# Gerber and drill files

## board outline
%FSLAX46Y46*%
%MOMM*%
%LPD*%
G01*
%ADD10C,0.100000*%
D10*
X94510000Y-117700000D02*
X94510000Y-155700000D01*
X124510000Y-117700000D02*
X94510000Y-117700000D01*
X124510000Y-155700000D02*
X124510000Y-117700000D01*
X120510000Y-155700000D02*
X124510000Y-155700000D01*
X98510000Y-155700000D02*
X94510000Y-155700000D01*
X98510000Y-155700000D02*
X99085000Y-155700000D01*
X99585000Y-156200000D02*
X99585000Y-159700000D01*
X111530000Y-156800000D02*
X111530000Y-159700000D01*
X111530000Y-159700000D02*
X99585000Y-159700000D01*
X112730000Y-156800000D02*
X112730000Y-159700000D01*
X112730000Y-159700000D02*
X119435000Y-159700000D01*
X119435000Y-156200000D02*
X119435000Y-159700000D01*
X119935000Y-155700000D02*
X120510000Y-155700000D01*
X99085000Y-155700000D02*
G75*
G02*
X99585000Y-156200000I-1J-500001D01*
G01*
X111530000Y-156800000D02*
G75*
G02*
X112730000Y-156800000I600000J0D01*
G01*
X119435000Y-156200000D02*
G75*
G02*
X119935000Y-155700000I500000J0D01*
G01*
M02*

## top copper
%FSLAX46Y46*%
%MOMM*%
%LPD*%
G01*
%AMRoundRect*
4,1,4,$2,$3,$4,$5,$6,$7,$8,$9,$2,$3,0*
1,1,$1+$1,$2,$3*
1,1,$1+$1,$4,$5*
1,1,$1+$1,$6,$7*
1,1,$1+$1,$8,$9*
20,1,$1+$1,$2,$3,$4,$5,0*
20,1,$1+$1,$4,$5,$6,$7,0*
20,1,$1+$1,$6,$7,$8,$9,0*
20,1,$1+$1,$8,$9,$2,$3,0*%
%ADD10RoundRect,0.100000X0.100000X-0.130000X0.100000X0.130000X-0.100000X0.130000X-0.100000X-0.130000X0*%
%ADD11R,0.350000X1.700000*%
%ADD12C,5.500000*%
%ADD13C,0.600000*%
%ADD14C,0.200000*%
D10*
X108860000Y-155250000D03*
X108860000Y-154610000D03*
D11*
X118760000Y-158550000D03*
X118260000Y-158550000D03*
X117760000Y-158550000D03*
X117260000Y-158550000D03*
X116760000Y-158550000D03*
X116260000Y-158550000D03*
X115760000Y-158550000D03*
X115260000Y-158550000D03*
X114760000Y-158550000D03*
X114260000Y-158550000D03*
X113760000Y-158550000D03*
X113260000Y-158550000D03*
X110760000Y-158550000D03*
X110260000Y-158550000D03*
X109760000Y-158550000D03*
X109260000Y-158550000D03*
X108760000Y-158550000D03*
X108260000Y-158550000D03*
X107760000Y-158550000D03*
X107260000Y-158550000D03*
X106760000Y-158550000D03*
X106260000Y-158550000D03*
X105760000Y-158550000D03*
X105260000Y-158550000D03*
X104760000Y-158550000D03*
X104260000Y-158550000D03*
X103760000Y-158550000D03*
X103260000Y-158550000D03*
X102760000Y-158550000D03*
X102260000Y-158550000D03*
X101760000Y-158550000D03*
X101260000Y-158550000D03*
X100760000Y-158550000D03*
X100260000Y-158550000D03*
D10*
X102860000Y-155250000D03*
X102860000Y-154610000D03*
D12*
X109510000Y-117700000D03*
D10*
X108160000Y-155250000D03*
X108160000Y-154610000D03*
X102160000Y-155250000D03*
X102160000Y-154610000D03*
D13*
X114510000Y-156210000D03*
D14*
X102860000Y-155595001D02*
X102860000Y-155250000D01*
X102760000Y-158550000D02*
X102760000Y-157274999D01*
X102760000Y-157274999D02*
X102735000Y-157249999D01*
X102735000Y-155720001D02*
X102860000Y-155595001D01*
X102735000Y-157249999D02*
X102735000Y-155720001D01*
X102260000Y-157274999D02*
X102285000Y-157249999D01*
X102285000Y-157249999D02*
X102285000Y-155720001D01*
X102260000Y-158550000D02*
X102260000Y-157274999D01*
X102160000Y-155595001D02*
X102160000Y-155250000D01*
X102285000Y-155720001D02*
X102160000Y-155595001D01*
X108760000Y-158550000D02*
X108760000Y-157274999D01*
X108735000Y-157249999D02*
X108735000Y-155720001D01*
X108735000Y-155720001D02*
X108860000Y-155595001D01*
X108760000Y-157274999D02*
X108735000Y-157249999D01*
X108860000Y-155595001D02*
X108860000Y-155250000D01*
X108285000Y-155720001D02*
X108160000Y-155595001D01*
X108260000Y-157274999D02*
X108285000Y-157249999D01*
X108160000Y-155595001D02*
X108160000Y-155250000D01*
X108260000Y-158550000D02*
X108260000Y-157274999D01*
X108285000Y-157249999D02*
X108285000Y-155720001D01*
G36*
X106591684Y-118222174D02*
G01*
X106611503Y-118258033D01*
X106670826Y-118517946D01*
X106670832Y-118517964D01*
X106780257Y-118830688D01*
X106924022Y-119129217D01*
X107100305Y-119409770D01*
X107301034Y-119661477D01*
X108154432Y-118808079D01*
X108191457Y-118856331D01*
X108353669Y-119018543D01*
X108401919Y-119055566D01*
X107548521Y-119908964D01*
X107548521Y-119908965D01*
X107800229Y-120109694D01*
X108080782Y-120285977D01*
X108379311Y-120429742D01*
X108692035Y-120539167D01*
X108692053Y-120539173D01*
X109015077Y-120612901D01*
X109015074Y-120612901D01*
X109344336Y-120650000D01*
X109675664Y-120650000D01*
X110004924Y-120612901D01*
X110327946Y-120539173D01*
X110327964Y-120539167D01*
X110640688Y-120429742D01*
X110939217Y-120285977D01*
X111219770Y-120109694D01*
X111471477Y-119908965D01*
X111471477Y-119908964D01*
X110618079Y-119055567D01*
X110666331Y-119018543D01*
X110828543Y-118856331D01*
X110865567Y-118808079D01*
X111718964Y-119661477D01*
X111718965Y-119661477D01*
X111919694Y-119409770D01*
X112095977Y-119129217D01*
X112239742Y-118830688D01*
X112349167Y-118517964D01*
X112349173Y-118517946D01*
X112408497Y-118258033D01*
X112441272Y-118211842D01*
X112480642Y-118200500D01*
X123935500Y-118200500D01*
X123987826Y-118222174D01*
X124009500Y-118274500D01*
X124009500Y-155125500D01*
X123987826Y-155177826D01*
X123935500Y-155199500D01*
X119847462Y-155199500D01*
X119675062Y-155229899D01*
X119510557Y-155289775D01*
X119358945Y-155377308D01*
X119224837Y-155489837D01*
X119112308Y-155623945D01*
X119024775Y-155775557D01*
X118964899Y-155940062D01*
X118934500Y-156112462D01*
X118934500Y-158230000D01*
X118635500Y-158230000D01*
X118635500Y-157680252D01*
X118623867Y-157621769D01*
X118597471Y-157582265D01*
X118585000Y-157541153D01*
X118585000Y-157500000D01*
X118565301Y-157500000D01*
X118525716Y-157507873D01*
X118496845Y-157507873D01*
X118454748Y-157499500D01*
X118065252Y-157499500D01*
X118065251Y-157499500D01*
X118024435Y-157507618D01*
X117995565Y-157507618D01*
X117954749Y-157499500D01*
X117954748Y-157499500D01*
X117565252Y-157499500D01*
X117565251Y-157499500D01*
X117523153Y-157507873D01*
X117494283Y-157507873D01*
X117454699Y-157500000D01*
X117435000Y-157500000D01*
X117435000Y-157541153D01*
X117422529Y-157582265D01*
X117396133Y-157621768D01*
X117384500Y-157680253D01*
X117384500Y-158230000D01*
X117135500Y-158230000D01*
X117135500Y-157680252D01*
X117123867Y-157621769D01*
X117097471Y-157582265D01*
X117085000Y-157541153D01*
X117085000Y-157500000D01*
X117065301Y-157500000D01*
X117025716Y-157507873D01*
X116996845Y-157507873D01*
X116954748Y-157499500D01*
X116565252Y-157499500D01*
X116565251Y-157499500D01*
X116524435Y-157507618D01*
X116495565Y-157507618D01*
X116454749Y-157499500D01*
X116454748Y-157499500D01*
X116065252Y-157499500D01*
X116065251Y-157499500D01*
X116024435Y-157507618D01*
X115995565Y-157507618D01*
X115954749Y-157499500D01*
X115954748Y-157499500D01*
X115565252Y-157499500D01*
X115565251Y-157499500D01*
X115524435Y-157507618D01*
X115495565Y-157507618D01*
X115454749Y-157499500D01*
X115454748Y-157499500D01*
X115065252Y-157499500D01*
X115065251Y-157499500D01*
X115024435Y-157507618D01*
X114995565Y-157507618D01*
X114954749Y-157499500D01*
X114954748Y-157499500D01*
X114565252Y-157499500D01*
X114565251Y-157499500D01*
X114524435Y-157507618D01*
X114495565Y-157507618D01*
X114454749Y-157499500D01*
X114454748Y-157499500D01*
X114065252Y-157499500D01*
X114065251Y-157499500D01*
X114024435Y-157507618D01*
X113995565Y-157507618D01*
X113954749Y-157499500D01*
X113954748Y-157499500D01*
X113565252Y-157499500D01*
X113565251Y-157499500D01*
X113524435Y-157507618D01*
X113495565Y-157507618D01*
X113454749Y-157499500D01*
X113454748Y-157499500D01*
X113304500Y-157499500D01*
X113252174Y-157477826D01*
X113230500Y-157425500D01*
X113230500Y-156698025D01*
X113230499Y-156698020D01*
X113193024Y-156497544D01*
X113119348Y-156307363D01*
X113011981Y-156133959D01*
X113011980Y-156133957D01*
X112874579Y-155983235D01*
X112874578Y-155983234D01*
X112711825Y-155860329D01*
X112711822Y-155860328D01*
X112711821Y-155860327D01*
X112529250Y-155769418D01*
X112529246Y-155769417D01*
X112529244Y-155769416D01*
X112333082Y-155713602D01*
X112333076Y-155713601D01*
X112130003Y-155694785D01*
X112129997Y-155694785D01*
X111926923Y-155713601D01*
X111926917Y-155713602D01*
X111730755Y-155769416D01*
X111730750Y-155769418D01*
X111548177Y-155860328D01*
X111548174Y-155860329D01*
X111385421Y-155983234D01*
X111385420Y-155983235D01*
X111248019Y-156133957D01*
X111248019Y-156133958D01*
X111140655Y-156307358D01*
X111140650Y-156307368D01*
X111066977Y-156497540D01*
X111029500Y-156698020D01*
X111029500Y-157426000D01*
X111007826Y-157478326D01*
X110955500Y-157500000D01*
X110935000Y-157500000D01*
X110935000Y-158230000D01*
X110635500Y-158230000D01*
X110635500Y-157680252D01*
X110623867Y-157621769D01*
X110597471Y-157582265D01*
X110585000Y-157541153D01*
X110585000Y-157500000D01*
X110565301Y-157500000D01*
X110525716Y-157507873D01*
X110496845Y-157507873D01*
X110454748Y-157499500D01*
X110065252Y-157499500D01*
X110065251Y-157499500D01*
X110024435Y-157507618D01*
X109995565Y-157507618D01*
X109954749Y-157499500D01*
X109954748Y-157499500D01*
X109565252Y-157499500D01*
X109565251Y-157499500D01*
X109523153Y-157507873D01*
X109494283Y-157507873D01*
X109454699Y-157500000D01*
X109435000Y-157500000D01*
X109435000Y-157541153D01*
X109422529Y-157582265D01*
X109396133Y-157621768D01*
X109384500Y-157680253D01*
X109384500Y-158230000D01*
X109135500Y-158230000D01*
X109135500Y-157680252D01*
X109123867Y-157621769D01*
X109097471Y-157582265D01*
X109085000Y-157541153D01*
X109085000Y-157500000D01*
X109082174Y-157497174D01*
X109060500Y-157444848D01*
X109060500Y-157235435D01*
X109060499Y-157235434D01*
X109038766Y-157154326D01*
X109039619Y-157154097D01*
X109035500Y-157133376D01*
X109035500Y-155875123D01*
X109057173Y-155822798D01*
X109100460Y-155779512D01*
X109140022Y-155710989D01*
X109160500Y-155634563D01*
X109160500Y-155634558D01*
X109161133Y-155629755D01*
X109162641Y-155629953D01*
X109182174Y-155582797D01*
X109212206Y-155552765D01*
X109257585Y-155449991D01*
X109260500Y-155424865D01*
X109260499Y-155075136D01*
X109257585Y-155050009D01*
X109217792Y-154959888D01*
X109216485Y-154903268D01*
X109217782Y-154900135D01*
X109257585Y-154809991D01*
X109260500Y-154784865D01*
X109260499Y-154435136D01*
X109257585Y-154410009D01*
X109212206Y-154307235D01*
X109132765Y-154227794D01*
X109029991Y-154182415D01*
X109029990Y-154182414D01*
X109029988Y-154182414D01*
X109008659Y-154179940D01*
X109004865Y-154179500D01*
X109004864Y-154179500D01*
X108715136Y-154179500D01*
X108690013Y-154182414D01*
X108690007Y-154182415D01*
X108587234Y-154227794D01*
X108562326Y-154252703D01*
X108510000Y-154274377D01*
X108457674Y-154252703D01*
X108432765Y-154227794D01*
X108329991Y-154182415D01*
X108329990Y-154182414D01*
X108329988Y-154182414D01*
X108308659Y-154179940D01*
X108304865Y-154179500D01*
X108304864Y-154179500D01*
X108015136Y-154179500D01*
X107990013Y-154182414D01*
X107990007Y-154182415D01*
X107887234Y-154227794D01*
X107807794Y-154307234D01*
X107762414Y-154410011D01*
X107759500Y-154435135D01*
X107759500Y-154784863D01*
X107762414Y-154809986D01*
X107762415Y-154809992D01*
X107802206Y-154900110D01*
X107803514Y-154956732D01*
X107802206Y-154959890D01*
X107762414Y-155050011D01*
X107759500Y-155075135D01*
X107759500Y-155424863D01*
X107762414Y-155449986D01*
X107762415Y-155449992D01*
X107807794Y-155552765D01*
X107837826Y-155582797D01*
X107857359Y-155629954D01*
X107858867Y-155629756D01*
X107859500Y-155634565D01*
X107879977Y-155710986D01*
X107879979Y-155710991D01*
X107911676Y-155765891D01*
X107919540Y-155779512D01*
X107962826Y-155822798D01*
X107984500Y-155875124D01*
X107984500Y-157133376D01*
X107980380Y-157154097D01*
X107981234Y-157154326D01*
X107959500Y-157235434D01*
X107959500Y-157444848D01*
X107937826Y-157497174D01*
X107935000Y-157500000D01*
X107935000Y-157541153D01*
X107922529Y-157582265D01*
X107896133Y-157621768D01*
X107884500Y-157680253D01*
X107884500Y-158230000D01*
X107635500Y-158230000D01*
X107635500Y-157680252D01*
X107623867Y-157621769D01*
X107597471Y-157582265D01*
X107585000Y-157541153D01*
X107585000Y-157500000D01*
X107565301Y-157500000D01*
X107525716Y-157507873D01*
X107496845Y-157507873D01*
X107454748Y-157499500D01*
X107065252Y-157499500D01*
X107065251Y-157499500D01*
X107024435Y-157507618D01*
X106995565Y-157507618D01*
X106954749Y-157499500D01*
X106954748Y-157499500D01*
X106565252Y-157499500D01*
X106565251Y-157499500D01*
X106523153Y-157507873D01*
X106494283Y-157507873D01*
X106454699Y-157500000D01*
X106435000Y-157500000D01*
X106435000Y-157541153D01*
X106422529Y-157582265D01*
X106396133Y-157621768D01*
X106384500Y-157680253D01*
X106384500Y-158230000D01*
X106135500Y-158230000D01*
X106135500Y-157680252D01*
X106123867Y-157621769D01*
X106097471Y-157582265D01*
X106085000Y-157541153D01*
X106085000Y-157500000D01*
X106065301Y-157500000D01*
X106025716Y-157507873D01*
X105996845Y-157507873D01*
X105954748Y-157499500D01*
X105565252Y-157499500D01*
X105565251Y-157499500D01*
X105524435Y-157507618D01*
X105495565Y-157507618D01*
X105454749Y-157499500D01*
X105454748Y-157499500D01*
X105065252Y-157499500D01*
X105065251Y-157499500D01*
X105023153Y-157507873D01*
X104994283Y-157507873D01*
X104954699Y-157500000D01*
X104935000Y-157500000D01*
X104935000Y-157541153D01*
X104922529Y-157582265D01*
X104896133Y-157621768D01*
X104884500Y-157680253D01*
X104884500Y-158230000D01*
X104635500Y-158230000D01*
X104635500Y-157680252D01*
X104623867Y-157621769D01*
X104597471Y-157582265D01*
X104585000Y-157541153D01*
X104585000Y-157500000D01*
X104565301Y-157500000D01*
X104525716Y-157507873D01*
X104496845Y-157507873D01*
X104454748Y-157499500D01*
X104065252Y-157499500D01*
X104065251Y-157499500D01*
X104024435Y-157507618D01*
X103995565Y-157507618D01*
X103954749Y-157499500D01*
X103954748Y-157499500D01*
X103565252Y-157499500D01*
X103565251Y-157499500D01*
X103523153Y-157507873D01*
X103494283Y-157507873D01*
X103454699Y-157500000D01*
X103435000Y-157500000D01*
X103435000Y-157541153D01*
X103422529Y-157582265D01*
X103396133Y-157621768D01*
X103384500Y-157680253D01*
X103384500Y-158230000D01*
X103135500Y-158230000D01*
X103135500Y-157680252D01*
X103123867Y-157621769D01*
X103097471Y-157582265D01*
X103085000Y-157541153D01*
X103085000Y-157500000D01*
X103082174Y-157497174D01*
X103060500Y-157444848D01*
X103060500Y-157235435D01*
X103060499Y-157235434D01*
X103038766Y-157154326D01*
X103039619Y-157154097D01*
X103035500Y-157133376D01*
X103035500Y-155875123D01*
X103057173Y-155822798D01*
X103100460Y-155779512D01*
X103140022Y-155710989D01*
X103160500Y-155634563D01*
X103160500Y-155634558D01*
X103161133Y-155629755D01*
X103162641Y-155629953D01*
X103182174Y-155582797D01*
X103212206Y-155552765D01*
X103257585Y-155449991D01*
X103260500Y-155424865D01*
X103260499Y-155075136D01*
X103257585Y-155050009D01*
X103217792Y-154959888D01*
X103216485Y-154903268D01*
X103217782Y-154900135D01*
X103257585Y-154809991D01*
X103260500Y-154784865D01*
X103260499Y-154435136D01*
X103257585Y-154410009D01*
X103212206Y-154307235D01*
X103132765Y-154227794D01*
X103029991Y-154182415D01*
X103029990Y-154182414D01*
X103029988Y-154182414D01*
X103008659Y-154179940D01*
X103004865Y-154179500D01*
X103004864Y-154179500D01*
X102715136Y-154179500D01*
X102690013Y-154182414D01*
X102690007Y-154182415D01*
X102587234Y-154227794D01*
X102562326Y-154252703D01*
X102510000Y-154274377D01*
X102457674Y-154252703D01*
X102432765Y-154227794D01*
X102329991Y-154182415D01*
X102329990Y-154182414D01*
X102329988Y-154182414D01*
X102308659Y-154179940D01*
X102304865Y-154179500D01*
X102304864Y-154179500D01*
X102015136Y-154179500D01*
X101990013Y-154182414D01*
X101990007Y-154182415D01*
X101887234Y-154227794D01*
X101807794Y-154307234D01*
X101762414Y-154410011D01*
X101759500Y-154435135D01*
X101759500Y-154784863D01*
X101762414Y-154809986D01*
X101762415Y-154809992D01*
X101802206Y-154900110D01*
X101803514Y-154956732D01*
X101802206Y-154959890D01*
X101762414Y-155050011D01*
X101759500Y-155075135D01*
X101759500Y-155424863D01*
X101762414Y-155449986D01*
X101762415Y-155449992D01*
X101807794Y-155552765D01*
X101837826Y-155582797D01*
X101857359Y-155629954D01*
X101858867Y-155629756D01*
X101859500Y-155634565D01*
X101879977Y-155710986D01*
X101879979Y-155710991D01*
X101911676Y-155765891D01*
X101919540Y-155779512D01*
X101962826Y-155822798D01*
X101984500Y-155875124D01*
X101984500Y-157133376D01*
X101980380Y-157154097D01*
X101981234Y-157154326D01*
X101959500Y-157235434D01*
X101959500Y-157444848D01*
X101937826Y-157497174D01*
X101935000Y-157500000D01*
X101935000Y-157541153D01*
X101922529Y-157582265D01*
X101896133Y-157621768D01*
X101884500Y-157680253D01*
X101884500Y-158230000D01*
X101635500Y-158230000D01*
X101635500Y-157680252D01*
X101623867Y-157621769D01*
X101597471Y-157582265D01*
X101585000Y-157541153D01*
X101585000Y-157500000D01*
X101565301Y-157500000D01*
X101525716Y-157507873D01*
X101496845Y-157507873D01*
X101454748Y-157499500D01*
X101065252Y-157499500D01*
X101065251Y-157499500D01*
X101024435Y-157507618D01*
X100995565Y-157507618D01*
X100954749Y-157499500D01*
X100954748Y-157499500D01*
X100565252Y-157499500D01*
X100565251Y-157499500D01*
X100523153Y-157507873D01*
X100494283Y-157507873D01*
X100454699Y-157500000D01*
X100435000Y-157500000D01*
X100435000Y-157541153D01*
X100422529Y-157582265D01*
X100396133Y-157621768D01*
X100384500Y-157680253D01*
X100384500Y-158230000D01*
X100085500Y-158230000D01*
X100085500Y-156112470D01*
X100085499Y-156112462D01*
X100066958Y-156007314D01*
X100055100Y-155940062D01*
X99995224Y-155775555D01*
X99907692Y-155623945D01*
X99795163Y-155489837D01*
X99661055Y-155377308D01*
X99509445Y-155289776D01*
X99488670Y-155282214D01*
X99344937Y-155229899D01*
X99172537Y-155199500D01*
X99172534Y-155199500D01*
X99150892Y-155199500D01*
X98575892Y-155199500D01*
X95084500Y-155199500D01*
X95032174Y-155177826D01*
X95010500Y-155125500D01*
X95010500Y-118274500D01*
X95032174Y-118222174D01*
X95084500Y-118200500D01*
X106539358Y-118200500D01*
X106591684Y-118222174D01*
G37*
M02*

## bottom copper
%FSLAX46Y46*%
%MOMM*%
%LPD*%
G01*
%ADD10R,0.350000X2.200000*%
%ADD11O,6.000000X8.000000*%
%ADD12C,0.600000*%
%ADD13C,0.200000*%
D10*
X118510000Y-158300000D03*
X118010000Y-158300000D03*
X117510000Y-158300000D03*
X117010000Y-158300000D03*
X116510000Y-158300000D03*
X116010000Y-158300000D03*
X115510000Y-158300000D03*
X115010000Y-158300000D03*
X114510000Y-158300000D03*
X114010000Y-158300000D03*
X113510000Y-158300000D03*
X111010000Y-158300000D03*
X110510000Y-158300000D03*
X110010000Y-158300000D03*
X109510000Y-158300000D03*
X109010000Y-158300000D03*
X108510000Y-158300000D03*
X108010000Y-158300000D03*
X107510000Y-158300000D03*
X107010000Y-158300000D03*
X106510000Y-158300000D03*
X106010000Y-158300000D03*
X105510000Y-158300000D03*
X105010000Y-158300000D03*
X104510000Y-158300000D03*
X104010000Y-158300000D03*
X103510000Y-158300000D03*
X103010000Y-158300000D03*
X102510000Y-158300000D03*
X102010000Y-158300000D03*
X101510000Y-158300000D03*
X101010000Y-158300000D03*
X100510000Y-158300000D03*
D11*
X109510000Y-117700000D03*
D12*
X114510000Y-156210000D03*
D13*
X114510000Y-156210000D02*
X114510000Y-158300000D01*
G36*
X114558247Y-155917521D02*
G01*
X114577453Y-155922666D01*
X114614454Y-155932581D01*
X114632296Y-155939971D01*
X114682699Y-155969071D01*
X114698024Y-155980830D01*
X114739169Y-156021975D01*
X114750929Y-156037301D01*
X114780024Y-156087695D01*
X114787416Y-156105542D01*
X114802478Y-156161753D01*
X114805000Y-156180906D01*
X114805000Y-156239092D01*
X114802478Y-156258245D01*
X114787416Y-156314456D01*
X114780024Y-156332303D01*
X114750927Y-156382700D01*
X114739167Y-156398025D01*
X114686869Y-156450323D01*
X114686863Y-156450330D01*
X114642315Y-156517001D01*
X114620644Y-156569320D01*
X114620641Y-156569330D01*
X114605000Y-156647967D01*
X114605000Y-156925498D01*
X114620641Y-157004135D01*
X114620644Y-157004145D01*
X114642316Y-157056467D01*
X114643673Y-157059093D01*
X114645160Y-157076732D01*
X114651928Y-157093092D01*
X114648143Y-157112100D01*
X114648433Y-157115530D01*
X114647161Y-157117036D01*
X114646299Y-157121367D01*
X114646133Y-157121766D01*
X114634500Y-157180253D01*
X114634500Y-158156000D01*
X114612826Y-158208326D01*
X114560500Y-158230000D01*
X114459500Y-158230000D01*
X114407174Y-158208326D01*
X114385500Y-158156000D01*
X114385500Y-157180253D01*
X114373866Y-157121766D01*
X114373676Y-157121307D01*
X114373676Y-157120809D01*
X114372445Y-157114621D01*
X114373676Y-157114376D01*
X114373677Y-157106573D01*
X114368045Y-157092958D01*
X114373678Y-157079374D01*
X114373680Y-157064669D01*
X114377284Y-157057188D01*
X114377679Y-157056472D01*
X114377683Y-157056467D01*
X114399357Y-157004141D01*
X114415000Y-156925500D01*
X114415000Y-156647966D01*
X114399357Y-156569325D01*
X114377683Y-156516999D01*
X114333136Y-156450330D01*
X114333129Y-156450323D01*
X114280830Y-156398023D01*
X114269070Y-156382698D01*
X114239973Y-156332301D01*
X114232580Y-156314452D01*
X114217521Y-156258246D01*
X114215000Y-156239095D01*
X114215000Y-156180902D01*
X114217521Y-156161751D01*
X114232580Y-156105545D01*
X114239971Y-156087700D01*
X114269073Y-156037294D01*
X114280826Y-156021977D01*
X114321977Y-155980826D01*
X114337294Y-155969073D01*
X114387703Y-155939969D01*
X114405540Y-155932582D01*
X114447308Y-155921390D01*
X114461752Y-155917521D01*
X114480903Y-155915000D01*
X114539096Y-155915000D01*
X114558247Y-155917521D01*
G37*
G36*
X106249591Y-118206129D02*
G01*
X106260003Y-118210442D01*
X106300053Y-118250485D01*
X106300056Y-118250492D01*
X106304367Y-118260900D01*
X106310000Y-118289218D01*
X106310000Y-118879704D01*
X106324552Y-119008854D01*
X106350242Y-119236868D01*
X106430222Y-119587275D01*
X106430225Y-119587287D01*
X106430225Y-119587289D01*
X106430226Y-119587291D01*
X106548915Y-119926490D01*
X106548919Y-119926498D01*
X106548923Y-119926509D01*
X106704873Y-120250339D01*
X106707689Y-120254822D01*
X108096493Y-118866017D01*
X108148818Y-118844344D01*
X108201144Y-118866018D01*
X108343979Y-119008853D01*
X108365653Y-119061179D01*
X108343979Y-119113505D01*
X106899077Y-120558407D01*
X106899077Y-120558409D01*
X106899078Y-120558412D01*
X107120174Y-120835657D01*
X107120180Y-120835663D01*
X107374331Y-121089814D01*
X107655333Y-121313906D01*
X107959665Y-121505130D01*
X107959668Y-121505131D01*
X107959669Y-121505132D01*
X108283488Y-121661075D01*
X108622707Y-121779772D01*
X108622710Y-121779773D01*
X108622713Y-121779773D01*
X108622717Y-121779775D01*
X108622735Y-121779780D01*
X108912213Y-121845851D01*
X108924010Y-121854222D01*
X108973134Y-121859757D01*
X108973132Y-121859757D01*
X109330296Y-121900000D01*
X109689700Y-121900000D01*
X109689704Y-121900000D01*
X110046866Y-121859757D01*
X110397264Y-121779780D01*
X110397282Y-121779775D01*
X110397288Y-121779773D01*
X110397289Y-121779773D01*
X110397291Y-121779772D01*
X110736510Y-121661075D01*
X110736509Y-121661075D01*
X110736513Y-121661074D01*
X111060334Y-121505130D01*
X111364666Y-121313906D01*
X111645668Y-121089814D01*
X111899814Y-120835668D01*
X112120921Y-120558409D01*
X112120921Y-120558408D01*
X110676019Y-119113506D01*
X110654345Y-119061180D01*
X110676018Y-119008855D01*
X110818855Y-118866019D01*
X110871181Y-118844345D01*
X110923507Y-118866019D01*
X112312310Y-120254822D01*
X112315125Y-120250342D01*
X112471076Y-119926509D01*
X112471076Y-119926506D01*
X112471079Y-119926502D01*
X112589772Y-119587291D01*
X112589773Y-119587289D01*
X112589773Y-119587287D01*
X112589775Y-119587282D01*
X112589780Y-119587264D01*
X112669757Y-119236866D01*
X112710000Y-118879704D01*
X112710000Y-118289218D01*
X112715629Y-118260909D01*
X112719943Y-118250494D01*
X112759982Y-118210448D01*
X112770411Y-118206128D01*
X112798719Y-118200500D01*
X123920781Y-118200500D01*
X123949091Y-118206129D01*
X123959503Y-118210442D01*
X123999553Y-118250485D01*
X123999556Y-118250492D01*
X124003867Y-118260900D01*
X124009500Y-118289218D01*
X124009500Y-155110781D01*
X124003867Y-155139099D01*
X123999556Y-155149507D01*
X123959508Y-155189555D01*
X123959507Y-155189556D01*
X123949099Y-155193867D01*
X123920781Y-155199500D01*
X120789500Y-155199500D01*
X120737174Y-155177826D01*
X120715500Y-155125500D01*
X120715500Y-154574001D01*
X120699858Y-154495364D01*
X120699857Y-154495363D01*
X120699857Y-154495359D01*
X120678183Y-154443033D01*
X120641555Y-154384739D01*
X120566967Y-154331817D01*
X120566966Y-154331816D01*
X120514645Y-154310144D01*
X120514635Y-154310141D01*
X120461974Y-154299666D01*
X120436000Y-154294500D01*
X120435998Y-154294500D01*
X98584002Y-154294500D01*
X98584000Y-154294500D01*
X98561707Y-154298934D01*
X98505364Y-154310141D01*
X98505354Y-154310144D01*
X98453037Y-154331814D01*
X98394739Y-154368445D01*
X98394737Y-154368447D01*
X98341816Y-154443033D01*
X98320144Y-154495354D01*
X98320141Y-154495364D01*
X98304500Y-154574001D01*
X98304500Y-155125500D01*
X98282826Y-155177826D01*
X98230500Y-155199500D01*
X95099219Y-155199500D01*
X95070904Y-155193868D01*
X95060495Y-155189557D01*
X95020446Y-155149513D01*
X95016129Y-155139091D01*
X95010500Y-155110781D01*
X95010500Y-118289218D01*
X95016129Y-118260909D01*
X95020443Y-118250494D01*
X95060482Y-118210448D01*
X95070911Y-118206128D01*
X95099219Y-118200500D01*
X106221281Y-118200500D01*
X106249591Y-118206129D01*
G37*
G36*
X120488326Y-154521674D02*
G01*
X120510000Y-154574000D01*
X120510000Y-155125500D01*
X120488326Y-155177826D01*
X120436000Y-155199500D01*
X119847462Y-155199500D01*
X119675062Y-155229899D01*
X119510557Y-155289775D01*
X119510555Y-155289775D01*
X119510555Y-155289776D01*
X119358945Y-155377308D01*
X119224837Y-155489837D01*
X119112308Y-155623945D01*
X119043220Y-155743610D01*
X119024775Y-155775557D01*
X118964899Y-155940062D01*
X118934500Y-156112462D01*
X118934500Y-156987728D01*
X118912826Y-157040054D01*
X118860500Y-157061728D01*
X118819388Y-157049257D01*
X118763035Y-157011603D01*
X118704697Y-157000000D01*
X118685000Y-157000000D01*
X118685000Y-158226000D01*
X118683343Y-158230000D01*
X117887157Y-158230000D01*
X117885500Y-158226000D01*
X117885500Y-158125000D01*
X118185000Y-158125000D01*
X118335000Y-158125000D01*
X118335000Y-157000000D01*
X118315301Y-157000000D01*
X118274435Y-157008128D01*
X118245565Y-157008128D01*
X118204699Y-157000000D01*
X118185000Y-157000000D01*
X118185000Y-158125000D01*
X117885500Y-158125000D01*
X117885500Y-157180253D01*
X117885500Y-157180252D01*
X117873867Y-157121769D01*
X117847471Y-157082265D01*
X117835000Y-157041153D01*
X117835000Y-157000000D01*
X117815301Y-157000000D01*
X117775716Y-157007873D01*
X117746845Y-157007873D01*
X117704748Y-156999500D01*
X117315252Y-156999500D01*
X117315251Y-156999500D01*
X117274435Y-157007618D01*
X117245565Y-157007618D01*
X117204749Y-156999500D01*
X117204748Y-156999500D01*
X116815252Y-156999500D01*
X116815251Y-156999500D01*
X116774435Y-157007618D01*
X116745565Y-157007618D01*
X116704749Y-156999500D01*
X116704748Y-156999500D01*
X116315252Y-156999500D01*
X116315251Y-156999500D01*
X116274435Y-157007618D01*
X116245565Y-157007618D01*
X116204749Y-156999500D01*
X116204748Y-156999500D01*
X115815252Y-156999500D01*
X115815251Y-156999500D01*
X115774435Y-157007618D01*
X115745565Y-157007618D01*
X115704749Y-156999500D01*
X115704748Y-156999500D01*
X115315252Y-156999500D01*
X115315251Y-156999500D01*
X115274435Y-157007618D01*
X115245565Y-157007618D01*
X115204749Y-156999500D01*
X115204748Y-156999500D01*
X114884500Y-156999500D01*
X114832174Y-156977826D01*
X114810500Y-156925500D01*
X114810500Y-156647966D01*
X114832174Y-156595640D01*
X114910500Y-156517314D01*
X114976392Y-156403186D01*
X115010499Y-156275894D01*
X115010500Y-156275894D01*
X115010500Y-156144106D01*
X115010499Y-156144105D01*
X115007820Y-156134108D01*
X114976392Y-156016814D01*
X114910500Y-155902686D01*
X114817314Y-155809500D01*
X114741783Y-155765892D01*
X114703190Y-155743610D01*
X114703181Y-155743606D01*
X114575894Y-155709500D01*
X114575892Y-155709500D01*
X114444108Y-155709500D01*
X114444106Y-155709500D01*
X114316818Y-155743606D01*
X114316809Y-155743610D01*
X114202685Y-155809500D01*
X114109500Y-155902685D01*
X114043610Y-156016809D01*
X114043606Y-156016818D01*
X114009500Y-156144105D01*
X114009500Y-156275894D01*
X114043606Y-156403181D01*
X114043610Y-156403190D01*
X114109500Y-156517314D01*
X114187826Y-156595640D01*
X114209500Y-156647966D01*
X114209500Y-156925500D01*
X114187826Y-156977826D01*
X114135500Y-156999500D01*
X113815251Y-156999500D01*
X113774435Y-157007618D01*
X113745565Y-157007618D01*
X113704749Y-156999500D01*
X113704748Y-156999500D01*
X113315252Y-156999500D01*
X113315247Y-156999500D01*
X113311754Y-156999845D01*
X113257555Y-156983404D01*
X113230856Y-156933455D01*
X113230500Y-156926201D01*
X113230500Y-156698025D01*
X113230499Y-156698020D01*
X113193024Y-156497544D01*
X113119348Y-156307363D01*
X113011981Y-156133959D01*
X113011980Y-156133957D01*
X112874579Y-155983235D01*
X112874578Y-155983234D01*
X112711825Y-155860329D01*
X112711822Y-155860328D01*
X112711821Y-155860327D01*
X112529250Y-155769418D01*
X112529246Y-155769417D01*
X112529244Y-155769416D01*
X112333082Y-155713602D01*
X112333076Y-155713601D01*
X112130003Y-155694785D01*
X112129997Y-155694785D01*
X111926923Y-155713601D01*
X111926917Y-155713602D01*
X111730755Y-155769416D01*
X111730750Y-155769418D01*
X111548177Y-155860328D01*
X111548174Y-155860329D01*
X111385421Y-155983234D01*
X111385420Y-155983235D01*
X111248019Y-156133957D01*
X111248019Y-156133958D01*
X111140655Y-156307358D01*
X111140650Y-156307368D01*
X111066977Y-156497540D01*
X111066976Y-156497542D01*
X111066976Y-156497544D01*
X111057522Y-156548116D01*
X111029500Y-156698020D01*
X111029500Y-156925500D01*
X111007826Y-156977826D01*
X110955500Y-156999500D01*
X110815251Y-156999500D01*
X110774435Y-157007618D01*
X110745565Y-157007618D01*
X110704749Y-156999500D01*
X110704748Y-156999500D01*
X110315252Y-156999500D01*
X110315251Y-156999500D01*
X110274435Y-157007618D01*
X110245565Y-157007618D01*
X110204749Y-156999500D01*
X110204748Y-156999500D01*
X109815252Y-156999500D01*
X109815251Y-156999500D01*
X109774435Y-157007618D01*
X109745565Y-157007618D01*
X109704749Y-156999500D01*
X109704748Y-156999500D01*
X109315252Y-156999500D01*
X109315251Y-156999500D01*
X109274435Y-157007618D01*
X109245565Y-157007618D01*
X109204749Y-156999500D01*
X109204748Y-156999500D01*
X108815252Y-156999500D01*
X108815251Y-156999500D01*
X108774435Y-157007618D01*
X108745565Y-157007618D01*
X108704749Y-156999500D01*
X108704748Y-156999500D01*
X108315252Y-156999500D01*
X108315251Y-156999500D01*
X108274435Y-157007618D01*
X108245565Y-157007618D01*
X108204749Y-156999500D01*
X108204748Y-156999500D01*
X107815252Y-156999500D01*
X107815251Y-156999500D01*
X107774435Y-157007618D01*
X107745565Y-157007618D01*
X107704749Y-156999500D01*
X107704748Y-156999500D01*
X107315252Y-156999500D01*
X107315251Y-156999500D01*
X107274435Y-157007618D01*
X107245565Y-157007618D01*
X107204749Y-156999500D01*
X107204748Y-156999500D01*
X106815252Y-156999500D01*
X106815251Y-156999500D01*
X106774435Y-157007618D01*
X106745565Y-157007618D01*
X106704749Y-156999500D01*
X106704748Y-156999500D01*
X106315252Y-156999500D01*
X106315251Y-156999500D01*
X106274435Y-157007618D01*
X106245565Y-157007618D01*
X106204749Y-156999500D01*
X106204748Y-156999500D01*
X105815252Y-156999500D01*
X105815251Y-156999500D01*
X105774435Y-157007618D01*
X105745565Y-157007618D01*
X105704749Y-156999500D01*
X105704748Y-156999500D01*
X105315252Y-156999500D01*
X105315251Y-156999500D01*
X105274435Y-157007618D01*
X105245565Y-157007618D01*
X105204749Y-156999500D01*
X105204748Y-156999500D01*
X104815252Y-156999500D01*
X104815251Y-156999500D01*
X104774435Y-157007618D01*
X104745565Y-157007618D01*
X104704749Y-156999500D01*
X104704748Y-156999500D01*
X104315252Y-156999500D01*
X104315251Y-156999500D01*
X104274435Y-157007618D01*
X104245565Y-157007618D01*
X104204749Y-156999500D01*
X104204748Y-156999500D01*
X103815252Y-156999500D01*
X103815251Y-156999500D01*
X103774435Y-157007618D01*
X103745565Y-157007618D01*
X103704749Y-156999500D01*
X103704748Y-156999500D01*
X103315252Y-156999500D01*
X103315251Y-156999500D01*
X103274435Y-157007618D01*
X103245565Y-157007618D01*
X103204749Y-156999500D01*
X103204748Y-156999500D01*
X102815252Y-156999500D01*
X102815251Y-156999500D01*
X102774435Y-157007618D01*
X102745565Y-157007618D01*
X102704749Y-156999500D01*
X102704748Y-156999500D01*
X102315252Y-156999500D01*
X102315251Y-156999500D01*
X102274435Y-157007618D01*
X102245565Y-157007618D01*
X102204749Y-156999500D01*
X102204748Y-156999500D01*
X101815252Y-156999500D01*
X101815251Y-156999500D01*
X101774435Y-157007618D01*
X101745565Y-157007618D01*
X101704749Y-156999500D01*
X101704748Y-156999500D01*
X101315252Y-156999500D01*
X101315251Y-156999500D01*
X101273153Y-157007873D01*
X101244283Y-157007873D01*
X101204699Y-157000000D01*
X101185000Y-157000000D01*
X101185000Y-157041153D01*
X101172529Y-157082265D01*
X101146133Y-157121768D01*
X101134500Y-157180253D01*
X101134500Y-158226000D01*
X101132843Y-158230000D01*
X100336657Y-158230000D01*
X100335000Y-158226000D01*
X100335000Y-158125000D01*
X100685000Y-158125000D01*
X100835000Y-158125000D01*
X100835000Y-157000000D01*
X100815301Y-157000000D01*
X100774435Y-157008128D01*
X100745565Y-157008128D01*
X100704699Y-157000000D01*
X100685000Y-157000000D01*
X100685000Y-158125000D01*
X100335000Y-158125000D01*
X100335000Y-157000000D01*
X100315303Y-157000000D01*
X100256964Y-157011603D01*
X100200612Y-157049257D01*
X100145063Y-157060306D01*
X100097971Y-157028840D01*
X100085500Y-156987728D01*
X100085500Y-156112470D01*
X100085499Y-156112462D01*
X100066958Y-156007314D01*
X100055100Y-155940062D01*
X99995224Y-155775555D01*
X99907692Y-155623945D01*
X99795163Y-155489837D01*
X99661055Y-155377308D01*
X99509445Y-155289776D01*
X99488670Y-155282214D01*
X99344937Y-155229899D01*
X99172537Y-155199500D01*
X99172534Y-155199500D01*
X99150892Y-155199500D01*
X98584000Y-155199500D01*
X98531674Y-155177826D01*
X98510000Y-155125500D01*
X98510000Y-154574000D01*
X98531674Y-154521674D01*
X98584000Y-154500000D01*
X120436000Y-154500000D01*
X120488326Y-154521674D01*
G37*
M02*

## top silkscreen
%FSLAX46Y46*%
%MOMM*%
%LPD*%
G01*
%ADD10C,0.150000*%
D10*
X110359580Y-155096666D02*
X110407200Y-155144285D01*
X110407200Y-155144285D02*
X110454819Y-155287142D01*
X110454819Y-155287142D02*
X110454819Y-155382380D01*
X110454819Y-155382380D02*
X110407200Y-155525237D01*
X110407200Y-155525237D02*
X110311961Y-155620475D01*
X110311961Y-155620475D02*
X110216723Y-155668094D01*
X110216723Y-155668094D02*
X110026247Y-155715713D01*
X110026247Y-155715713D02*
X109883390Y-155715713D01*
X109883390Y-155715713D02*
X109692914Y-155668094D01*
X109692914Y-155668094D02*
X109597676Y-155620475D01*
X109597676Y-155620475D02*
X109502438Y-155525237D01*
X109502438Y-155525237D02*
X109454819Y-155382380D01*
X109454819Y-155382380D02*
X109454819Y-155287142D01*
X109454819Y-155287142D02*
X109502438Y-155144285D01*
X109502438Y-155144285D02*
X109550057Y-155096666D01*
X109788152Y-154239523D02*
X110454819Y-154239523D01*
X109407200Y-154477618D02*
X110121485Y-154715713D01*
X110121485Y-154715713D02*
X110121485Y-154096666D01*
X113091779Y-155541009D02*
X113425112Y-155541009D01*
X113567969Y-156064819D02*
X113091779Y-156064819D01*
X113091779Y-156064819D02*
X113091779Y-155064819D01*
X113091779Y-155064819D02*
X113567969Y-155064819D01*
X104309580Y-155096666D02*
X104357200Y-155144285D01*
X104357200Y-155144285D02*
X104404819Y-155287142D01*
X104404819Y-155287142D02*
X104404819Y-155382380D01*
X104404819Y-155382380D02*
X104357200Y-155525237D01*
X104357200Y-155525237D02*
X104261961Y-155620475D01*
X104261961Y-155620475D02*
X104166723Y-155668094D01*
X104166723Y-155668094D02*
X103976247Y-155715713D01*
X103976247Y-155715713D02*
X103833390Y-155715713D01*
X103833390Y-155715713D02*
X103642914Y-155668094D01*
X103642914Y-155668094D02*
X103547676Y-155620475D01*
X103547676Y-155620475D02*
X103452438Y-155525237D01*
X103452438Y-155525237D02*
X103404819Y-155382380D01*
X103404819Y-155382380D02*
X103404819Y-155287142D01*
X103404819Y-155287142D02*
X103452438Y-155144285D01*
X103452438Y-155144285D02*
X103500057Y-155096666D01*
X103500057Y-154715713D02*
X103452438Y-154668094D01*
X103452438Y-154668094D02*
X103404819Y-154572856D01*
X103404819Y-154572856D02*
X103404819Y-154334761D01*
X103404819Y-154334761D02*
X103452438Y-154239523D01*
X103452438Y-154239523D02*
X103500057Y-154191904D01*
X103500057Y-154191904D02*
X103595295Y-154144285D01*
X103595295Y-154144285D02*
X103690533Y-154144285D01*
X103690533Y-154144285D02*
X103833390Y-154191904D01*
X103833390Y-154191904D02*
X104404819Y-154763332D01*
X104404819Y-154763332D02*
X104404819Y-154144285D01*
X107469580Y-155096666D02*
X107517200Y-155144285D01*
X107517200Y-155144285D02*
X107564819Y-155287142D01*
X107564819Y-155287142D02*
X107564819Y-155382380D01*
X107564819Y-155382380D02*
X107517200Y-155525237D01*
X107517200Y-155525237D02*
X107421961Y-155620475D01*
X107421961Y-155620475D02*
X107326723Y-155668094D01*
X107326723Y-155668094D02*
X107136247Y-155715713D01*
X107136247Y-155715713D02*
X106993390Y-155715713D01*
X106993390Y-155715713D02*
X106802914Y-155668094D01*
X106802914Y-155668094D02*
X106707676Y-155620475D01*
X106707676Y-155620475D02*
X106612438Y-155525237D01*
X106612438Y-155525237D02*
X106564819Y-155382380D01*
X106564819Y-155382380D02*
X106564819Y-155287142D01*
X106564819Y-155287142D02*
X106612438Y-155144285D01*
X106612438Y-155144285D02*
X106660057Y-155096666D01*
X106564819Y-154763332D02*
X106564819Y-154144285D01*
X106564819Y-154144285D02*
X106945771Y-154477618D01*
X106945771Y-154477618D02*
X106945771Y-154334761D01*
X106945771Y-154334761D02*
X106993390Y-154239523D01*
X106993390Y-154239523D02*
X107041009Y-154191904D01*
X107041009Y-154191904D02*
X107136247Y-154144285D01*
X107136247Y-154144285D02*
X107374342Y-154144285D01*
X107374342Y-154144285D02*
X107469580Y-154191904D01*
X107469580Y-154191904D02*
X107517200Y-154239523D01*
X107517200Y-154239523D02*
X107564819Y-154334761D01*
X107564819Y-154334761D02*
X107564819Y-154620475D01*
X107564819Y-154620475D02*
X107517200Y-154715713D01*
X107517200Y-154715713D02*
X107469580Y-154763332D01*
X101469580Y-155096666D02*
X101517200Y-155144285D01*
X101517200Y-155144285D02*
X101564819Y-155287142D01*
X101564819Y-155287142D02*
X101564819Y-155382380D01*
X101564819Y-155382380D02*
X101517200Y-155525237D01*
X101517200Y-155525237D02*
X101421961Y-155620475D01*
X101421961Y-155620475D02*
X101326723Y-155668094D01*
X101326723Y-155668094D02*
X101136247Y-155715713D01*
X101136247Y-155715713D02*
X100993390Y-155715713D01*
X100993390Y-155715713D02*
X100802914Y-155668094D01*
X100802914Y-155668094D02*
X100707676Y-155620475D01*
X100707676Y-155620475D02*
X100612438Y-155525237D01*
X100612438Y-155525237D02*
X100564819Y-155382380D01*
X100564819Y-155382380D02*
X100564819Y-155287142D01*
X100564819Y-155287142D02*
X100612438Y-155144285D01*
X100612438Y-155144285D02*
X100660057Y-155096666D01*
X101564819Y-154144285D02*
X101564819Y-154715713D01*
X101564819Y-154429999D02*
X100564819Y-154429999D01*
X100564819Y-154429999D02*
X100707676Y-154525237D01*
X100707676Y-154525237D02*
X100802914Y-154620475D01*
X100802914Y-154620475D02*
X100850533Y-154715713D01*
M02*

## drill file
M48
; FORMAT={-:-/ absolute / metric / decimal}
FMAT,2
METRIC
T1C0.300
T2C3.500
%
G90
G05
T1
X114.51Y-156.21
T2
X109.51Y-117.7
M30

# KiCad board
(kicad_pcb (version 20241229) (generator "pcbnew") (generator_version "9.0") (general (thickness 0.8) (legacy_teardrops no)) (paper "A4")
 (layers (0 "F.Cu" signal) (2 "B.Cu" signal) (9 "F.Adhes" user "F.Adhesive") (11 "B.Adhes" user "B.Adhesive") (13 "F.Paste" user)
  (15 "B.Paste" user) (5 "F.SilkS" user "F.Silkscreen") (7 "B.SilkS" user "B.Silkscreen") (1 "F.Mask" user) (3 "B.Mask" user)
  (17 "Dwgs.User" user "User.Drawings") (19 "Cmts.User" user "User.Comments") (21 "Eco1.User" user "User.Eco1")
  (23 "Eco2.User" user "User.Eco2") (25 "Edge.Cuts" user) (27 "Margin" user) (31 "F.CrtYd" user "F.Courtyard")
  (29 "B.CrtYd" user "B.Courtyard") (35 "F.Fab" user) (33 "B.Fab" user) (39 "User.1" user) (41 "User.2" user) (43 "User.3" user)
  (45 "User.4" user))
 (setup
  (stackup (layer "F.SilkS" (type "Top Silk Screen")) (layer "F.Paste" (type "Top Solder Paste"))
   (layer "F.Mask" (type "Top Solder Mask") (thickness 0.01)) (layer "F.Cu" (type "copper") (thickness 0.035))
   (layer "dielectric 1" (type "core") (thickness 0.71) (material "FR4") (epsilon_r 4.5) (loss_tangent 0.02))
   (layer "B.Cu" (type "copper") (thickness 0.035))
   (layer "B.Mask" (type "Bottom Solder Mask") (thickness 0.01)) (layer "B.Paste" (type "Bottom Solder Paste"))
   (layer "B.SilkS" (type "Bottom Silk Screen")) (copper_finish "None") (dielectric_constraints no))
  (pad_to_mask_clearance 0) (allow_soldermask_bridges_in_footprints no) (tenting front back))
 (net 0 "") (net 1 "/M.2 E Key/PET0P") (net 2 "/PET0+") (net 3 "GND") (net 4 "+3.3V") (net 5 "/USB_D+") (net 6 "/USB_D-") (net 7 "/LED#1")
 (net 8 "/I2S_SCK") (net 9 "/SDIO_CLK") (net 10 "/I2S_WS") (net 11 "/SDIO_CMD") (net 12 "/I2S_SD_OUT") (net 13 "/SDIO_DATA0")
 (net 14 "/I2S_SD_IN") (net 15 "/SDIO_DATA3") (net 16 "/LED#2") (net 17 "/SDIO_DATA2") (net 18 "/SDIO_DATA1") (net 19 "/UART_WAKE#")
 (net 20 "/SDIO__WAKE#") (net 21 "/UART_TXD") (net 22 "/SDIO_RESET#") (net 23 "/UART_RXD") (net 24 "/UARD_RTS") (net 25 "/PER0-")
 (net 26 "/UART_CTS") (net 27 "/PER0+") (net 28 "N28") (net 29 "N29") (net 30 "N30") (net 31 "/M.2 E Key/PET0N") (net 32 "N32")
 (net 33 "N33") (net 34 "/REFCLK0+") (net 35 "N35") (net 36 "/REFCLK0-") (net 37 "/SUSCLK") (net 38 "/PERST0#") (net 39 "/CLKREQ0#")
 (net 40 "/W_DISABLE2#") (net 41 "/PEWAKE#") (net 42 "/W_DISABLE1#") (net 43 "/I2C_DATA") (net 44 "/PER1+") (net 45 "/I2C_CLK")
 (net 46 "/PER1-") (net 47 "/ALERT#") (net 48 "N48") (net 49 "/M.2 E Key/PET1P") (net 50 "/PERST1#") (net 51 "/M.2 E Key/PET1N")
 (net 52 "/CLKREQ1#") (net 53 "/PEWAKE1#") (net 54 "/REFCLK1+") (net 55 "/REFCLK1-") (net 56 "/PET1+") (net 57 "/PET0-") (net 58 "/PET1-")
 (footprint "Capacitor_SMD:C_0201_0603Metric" (layer "F.Cu") (at 108.86 154.93 90)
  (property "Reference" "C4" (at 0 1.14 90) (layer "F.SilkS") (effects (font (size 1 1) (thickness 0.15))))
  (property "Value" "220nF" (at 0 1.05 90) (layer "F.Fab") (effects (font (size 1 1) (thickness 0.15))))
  (pad "" smd roundrect (at -0.345 0 90) (size 0.318 0.36) (layers "F.Paste") (roundrect_rratio 0.25))
  (pad "" smd roundrect (at 0.345 0 90) (size 0.318 0.36) (layers "F.Paste") (roundrect_rratio 0.25))
  (pad "1" smd roundrect (at -0.32 0 90) (size 0.46 0.4) (layers "F.Cu" "F.Mask") (roundrect_rratio 0.25) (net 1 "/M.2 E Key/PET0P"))
  (pad "2" smd roundrect (at 0.32 0 90) (size 0.46 0.4) (layers "F.Cu" "F.Mask") (roundrect_rratio 0.25) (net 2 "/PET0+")))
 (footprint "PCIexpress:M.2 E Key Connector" (layer "F.Cu") (at 109.51 158.59)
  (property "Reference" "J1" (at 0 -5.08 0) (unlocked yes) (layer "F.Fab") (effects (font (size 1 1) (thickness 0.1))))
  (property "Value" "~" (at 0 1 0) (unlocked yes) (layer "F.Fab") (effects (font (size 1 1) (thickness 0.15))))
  (fp_line (start -11 -2.89) (end -10.425 -2.89) (stroke (width 0.1) (type default)) (layer "Edge.Cuts"))
  (fp_line (start -9.925 -2.39) (end -9.925 1.11) (stroke (width 0.1) (type default)) (layer "Edge.Cuts"))
  (fp_line (start 2.02 -1.79) (end 2.02 1.11) (stroke (width 0.1) (type default)) (layer "Edge.Cuts"))
  (fp_line (start 2.02 1.11) (end -9.925 1.11) (stroke (width 0.1) (type default)) (layer "Edge.Cuts"))
  (fp_line (start 3.22 -1.79) (end 3.22 1.11) (stroke (width 0.1) (type default)) (layer "Edge.Cuts"))
  (fp_line (start 3.22 1.11) (end 9.925 1.11) (stroke (width 0.1) (type default)) (layer "Edge.Cuts"))
  (fp_line (start 9.925 -2.39) (end 9.925 1.11) (stroke (width 0.1) (type default)) (layer "Edge.Cuts"))
  (fp_line (start 10.425 -2.89) (end 11 -2.89) (stroke (width 0.1) (type default)) (layer "Edge.Cuts"))
  (fp_arc (start -10.425 -2.89) (mid -10.071447 -2.743553) (end -9.925 -2.39) (stroke (width 0.1) (type default)) (layer "Edge.Cuts"))
  (fp_arc (start 2.02 -1.79) (mid 2.62 -2.39) (end 3.22 -1.79) (stroke (width 0.1) (type default)) (layer "Edge.Cuts"))
  (fp_arc (start 9.925 -2.39) (mid 10.071447 -2.743553) (end 10.425 -2.89) (stroke (width 0.1) (type default)) (layer "Edge.Cuts"))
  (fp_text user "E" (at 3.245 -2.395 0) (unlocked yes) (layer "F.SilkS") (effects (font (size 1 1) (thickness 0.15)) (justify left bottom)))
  (pad "1" smd rect (at 9.25 -0.04 180) (size 0.35 1.7) (layers "F.Cu") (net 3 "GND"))
  (pad "2" smd rect (at 9 -0.29 180) (size 0.35 2.2) (layers "B.Cu") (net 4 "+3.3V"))
  (pad "3" smd rect (at 8.75 -0.04 180) (size 0.35 1.7) (layers "F.Cu") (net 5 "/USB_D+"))
  (pad "4" smd rect (at 8.5 -0.29 180) (size 0.35 2.2) (layers "B.Cu") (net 4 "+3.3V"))
  (pad "5" smd rect (at 8.25 -0.04 180) (size 0.35 1.7) (layers "F.Cu") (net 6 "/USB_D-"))
  (pad "6" smd rect (at 8 -0.29 180) (size 0.35 2.2) (layers "B.Cu") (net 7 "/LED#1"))
  (pad "7" smd rect (at 7.75 -0.04 180) (size 0.35 1.7) (layers "F.Cu") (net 3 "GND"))
  (pad "8" smd rect (at 7.5 -0.29 180) (size 0.35 2.2) (layers "B.Cu") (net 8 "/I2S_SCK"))
  (pad "9" smd rect (at 7.25 -0.04 180) (size 0.35 1.7) (layers "F.Cu") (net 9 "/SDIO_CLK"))
  (pad "10" smd rect (at 7 -0.29 180) (size 0.35 2.2) (layers "B.Cu") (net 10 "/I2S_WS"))
  (pad "11" smd rect (at 6.75 -0.04 180) (size 0.35 1.7) (layers "F.Cu") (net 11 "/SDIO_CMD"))
  (pad "12" smd rect (at 6.5 -0.29 180) (size 0.35 2.2) (layers "B.Cu") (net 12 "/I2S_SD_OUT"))
  (pad "13" smd rect (at 6.25 -0.04 180) (size 0.35 1.7) (layers "F.Cu") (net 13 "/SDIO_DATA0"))
  (pad "14" smd rect (at 6 -0.29 180) (size 0.35 2.2) (layers "B.Cu") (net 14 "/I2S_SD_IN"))
  (pad "15" smd rect (at 5.75 -0.04 180) (size 0.35 1.7) (layers "F.Cu") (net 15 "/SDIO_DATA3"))
  (pad "16" smd rect (at 5.5 -0.29 180) (size 0.35 2.2) (layers "B.Cu") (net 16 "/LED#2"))
  (pad "17" smd rect (at 5.25 -0.04 180) (size 0.35 1.7) (layers "F.Cu") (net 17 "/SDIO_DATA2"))
  (pad "18" smd rect (at 5 -0.29 180) (size 0.35 2.2) (layers "B.Cu") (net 3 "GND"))
  (pad "19" smd rect (at 4.75 -0.04 180) (size 0.35 1.7) (layers "F.Cu") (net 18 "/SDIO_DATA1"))
  (pad "20" smd rect (at 4.5 -0.29 180) (size 0.35 2.2) (layers "B.Cu") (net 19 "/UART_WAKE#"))
  (pad "21" smd rect (at 4.25 -0.04 180) (size 0.35 1.7) (layers "F.Cu") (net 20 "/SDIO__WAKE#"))
  (pad "22" smd rect (at 4 -0.29 180) (size 0.35 2.2) (layers "B.Cu") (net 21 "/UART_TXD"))
  (pad "23" smd rect (at 3.75 -0.04 180) (size 0.35 1.7) (layers "F.Cu") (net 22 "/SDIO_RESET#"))
  (pad "32" smd rect (at 1.5 -0.29 180) (size 0.35 2.2) (layers "B.Cu") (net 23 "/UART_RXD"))
  (pad "33" smd rect (at 1.25 -0.04 180) (size 0.35 1.7) (layers "F.Cu") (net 3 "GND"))
  (pad "34" smd rect (at 1 -0.29 180) (size 0.35 2.2) (layers "B.Cu") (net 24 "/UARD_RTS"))
  (pad "35" smd rect (at 0.75 -0.04 180) (size 0.35 1.7) (layers "F.Cu") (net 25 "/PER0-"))
  (pad "36" smd rect (at 0.5 -0.29 180) (size 0.35 2.2) (layers "B.Cu") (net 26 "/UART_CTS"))
  (pad "37" smd rect (at 0.25 -0.04 180) (size 0.35 1.7) (layers "F.Cu") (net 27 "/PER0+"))
  (pad "38" smd rect (at 0 -0.29 180) (size 0.35 2.2) (layers "B.Cu") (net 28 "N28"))
  (pad "39" smd rect (at -0.25 -0.04 180) (size 0.35 1.7) (layers "F.Cu") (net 3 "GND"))
  (pad "40" smd rect (at -0.5 -0.29 180) (size 0.35 2.2) (layers "B.Cu") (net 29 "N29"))
  (pad "41" smd rect (at -0.75 -0.04 180) (size 0.35 1.7) (layers "F.Cu") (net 1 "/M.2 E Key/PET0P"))
  (pad "42" smd rect (at -1 -0.29 180) (size 0.35 2.2) (layers "B.Cu") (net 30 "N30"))
  (pad "43" smd rect (at -1.25 -0.04 180) (size 0.35 1.7) (layers "F.Cu") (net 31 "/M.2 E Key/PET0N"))
  (pad "44" smd rect (at -1.5 -0.29 180) (size 0.35 2.2) (layers "B.Cu") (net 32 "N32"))
  (pad "45" smd rect (at -1.75 -0.04 180) (size 0.35 1.7) (layers "F.Cu") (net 3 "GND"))
  (pad "46" smd rect (at -2 -0.29 180) (size 0.35 2.2) (layers "B.Cu") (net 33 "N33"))
  (pad "47" smd rect (at -2.25 -0.04 180) (size 0.35 1.7) (layers "F.Cu") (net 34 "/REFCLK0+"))
  (pad "48" smd rect (at -2.5 -0.29 180) (size 0.35 2.2) (layers "B.Cu") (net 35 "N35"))
  (pad "49" smd rect (at -2.75 -0.04 180) (size 0.35 1.7) (layers "F.Cu") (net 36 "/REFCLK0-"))
  (pad "50" smd rect (at -3 -0.29 180) (size 0.35 2.2) (layers "B.Cu") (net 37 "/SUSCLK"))
  (pad "51" smd rect (at -3.25 -0.04 180) (size 0.35 1.7) (layers "F.Cu") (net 3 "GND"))
  (pad "52" smd rect (at -3.5 -0.29 180) (size 0.35 2.2) (layers "B.Cu") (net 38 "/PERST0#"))
  (pad "53" smd rect (at -3.75 -0.04 180) (size 0.35 1.7) (layers "F.Cu") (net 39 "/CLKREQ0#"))
  (pad "54" smd rect (at -4 -0.29 180) (size 0.35 2.2) (layers "B.Cu") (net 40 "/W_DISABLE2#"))
  (pad "55" smd rect (at -4.25 -0.04 180) (size 0.35 1.7) (layers "F.Cu") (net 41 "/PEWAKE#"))
  (pad "56" smd rect (at -4.5 -0.29 180) (size 0.35 2.2) (layers "B.Cu") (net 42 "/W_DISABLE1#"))
  (pad "57" smd rect (at -4.75 -0.04 180) (size 0.35 1.7) (layers "F.Cu") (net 3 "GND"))
  (pad "58" smd rect (at -5 -0.29 180) (size 0.35 2.2) (layers "B.Cu") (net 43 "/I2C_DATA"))
  (pad "59" smd rect (at -5.25 -0.04 180) (size 0.35 1.7) (layers "F.Cu") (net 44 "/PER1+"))
  (pad "60" smd rect (at -5.5 -0.29 180) (size 0.35 2.2) (layers "B.Cu") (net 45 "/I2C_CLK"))
  (pad "61" smd rect (at -5.75 -0.04 180) (size 0.35 1.7) (layers "F.Cu") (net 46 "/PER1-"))
  (pad "62" smd rect (at -6 -0.29 180) (size 0.35 2.2) (layers "B.Cu") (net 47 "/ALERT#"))
  (pad "63" smd rect (at -6.25 -0.04 180) (size 0.35 1.7) (layers "F.Cu") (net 3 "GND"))
  (pad "64" smd rect (at -6.5 -0.29 180) (size 0.35 2.2) (layers "B.Cu") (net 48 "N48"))
  (pad "65" smd rect (at -6.75 -0.04 180) (size 0.35 1.7) (layers "F.Cu") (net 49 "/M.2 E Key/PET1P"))
  (pad "66" smd rect (at -7 -0.29 180) (size 0.35 2.2) (layers "B.Cu") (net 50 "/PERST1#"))
  (pad "67" smd rect (at -7.25 -0.04 180) (size 0.35 1.7) (layers "F.Cu") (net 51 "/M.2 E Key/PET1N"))
  (pad "68" smd rect (at -7.5 -0.29 180) (size 0.35 2.2) (layers "B.Cu") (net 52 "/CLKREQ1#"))
  (pad "69" smd rect (at -7.75 -0.04 180) (size 0.35 1.7) (layers "F.Cu") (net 3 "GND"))
  (pad "70" smd rect (at -8 -0.29 180) (size 0.35 2.2) (layers "B.Cu") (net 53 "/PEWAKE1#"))
  (pad "71" smd rect (at -8.25 -0.04 180) (size 0.35 1.7) (layers "F.Cu") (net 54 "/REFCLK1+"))
  (pad "72" smd rect (at -8.5 -0.29 180) (size 0.35 2.2) (layers "B.Cu") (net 4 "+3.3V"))
  (pad "73" smd rect (at -8.75 -0.04 180) (size 0.35 1.7) (layers "F.Cu") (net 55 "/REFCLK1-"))
  (pad "74" smd rect (at -9 -0.29 180) (size 0.35 2.2) (layers "B.Cu") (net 4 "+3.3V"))
  (pad "75" smd rect (at -9.25 -0.04 180) (size 0.35 1.7) (layers "F.Cu") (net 3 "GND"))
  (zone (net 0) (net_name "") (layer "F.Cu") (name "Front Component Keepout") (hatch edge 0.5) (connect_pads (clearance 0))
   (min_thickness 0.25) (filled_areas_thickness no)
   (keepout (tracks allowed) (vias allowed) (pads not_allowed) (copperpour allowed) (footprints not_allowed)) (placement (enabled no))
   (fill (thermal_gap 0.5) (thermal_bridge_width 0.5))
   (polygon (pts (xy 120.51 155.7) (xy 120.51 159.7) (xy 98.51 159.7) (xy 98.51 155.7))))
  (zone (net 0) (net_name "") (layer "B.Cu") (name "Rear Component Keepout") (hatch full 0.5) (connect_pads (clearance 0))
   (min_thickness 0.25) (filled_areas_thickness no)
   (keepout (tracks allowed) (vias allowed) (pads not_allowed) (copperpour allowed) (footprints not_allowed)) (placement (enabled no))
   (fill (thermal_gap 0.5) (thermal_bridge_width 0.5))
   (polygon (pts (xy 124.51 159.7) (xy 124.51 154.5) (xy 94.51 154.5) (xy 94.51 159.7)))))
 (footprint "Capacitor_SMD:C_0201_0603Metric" (layer "F.Cu") (at 102.86 154.93 90)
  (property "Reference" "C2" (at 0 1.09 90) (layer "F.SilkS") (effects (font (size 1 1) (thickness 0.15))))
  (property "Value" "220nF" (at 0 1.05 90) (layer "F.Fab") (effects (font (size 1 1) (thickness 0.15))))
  (pad "" smd roundrect (at -0.345 0 90) (size 0.318 0.36) (layers "F.Paste") (roundrect_rratio 0.25))
  (pad "" smd roundrect (at 0.345 0 90) (size 0.318 0.36) (layers "F.Paste") (roundrect_rratio 0.25))
  (pad "1" smd roundrect (at -0.32 0 90) (size 0.46 0.4) (layers "F.Cu" "F.Mask") (roundrect_rratio 0.25) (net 49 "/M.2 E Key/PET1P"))
  (pad "2" smd roundrect (at 0.32 0 90) (size 0.46 0.4) (layers "F.Cu" "F.Mask") (roundrect_rratio 0.25) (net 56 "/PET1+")))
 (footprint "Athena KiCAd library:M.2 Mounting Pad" (layer "F.Cu") (at 109.51 117.7)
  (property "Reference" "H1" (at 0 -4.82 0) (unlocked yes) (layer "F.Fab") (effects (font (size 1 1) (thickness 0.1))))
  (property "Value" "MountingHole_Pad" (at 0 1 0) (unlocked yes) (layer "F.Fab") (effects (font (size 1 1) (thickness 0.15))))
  (pad "1" thru_hole circle (at 0 0) (size 5.5 5.5) (drill 3.5) (layers "*.Cu" "*.Mask") (remove_unused_layers no) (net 3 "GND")
   (padstack (mode front_inner_back)
    (layer "Inner" (shape circle) (size 5.5 5.5) (zone_connect -1))
    (layer "B.Cu" (shape oval) (size 6 8) (thermal_bridge_angle 45) (zone_connect -1)))))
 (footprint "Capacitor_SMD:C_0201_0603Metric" (layer "F.Cu") (at 108.16 154.93 90)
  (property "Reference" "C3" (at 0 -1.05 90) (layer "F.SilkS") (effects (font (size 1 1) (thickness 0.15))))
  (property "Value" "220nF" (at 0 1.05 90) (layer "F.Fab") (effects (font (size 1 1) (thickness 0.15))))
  (pad "" smd roundrect (at -0.345 0 90) (size 0.318 0.36) (layers "F.Paste") (roundrect_rratio 0.25))
  (pad "" smd roundrect (at 0.345 0 90) (size 0.318 0.36) (layers "F.Paste") (roundrect_rratio 0.25))
  (pad "1" smd roundrect (at -0.32 0 90) (size 0.46 0.4) (layers "F.Cu" "F.Mask") (roundrect_rratio 0.25) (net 31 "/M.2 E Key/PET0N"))
  (pad "2" smd roundrect (at 0.32 0 90) (size 0.46 0.4) (layers "F.Cu" "F.Mask") (roundrect_rratio 0.25) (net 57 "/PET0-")))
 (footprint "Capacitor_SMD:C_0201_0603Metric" (layer "F.Cu") (at 102.16 154.93 90)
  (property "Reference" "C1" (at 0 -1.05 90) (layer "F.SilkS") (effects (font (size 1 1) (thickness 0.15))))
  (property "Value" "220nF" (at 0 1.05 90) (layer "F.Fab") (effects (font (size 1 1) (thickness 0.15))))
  (pad "" smd roundrect (at -0.345 0 90) (size 0.318 0.36) (layers "F.Paste") (roundrect_rratio 0.25))
  (pad "" smd roundrect (at 0.345 0 90) (size 0.318 0.36) (layers "F.Paste") (roundrect_rratio 0.25))
  (pad "1" smd roundrect (at -0.32 0 90) (size 0.46 0.4) (layers "F.Cu" "F.Mask") (roundrect_rratio 0.25) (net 51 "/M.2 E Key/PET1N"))
  (pad "2" smd roundrect (at 0.32 0 90) (size 0.46 0.4) (layers "F.Cu" "F.Mask") (roundrect_rratio 0.25) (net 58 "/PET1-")))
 (gr_line (start 94.51 117.7) (end 94.51 155.7) (stroke (width 0.1) (type default)) (layer "Edge.Cuts"))
 (gr_line (start 124.51 117.7) (end 94.51 117.7) (stroke (width 0.1) (type default)) (layer "Edge.Cuts"))
 (gr_line (start 124.51 155.7) (end 124.51 117.7) (stroke (width 0.1) (type default)) (layer "Edge.Cuts"))
 (gr_line (start 120.51 155.7) (end 124.51 155.7) (stroke (width 0.1) (type default)) (layer "Edge.Cuts"))
 (gr_line (start 98.51 155.7) (end 94.51 155.7) (stroke (width 0.1) (type default)) (layer "Edge.Cuts"))
 (segment (start 102.86 155.595001) (end 102.86 155.25) (width 0.2) (layer "F.Cu") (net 49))
 (segment (start 102.76 158.55) (end 102.76 157.274999) (width 0.2) (layer "F.Cu") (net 49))
 (segment (start 102.76 157.274999) (end 102.735 157.249999) (width 0.2) (layer "F.Cu") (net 49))
 (segment (start 102.735 155.720001) (end 102.86 155.595001) (width 0.2) (layer "F.Cu") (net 49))
 (segment (start 102.735 157.249999) (end 102.735 155.720001) (width 0.2) (layer "F.Cu") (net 49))
 (segment (start 102.26 157.274999) (end 102.285 157.249999) (width 0.2) (layer "F.Cu") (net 51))
 (segment (start 102.285 157.249999) (end 102.285 155.720001) (width 0.2) (layer "F.Cu") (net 51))
 (segment (start 102.26 158.55) (end 102.26 157.274999) (width 0.2) (layer "F.Cu") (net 51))
 (segment (start 102.16 155.595001) (end 102.16 155.25) (width 0.2) (layer "F.Cu") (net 51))
 (segment (start 102.285 155.720001) (end 102.16 155.595001) (width 0.2) (layer "F.Cu") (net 51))
 (segment (start 108.76 158.55) (end 108.76 157.274999) (width 0.2) (layer "F.Cu") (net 1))
 (segment (start 108.735 157.249999) (end 108.735 155.720001) (width 0.2) (layer "F.Cu") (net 1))
 (segment (start 108.735 155.720001) (end 108.86 155.595001) (width 0.2) (layer "F.Cu") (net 1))
 (segment (start 108.76 157.274999) (end 108.735 157.249999) (width 0.2) (layer "F.Cu") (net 1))
 (segment (start 108.86 155.595001) (end 108.86 155.25) (width 0.2) (layer "F.Cu") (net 1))
 (segment (start 108.285 155.720001) (end 108.16 155.595001) (width 0.2) (layer "F.Cu") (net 31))
 (segment (start 108.26 157.274999) (end 108.285 157.249999) (width 0.2) (layer "F.Cu") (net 31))
 (segment (start 108.16 155.595001) (end 108.16 155.25) (width 0.2) (layer "F.Cu") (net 31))
 (segment (start 108.26 158.55) (end 108.26 157.274999) (width 0.2) (layer "F.Cu") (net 31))
 (segment (start 108.285 157.249999) (end 108.285 155.720001) (width 0.2) (layer "F.Cu") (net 31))
 (via (at 114.51 156.21) (size 0.6) (drill 0.3) (layers "F.Cu" "B.Cu") (free yes) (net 3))
 (segment (start 114.51 156.21) (end 114.51 158.3) (width 0.2) (layer "B.Cu") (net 3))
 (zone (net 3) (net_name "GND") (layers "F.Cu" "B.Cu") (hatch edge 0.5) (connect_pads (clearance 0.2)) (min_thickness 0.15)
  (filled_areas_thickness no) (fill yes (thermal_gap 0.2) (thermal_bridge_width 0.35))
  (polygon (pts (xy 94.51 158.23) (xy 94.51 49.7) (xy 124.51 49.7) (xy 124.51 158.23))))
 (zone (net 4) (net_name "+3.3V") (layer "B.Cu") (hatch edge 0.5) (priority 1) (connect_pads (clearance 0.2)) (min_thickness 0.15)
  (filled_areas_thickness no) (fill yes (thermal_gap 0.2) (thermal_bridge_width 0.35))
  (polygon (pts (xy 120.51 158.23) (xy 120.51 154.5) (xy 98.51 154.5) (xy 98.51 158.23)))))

